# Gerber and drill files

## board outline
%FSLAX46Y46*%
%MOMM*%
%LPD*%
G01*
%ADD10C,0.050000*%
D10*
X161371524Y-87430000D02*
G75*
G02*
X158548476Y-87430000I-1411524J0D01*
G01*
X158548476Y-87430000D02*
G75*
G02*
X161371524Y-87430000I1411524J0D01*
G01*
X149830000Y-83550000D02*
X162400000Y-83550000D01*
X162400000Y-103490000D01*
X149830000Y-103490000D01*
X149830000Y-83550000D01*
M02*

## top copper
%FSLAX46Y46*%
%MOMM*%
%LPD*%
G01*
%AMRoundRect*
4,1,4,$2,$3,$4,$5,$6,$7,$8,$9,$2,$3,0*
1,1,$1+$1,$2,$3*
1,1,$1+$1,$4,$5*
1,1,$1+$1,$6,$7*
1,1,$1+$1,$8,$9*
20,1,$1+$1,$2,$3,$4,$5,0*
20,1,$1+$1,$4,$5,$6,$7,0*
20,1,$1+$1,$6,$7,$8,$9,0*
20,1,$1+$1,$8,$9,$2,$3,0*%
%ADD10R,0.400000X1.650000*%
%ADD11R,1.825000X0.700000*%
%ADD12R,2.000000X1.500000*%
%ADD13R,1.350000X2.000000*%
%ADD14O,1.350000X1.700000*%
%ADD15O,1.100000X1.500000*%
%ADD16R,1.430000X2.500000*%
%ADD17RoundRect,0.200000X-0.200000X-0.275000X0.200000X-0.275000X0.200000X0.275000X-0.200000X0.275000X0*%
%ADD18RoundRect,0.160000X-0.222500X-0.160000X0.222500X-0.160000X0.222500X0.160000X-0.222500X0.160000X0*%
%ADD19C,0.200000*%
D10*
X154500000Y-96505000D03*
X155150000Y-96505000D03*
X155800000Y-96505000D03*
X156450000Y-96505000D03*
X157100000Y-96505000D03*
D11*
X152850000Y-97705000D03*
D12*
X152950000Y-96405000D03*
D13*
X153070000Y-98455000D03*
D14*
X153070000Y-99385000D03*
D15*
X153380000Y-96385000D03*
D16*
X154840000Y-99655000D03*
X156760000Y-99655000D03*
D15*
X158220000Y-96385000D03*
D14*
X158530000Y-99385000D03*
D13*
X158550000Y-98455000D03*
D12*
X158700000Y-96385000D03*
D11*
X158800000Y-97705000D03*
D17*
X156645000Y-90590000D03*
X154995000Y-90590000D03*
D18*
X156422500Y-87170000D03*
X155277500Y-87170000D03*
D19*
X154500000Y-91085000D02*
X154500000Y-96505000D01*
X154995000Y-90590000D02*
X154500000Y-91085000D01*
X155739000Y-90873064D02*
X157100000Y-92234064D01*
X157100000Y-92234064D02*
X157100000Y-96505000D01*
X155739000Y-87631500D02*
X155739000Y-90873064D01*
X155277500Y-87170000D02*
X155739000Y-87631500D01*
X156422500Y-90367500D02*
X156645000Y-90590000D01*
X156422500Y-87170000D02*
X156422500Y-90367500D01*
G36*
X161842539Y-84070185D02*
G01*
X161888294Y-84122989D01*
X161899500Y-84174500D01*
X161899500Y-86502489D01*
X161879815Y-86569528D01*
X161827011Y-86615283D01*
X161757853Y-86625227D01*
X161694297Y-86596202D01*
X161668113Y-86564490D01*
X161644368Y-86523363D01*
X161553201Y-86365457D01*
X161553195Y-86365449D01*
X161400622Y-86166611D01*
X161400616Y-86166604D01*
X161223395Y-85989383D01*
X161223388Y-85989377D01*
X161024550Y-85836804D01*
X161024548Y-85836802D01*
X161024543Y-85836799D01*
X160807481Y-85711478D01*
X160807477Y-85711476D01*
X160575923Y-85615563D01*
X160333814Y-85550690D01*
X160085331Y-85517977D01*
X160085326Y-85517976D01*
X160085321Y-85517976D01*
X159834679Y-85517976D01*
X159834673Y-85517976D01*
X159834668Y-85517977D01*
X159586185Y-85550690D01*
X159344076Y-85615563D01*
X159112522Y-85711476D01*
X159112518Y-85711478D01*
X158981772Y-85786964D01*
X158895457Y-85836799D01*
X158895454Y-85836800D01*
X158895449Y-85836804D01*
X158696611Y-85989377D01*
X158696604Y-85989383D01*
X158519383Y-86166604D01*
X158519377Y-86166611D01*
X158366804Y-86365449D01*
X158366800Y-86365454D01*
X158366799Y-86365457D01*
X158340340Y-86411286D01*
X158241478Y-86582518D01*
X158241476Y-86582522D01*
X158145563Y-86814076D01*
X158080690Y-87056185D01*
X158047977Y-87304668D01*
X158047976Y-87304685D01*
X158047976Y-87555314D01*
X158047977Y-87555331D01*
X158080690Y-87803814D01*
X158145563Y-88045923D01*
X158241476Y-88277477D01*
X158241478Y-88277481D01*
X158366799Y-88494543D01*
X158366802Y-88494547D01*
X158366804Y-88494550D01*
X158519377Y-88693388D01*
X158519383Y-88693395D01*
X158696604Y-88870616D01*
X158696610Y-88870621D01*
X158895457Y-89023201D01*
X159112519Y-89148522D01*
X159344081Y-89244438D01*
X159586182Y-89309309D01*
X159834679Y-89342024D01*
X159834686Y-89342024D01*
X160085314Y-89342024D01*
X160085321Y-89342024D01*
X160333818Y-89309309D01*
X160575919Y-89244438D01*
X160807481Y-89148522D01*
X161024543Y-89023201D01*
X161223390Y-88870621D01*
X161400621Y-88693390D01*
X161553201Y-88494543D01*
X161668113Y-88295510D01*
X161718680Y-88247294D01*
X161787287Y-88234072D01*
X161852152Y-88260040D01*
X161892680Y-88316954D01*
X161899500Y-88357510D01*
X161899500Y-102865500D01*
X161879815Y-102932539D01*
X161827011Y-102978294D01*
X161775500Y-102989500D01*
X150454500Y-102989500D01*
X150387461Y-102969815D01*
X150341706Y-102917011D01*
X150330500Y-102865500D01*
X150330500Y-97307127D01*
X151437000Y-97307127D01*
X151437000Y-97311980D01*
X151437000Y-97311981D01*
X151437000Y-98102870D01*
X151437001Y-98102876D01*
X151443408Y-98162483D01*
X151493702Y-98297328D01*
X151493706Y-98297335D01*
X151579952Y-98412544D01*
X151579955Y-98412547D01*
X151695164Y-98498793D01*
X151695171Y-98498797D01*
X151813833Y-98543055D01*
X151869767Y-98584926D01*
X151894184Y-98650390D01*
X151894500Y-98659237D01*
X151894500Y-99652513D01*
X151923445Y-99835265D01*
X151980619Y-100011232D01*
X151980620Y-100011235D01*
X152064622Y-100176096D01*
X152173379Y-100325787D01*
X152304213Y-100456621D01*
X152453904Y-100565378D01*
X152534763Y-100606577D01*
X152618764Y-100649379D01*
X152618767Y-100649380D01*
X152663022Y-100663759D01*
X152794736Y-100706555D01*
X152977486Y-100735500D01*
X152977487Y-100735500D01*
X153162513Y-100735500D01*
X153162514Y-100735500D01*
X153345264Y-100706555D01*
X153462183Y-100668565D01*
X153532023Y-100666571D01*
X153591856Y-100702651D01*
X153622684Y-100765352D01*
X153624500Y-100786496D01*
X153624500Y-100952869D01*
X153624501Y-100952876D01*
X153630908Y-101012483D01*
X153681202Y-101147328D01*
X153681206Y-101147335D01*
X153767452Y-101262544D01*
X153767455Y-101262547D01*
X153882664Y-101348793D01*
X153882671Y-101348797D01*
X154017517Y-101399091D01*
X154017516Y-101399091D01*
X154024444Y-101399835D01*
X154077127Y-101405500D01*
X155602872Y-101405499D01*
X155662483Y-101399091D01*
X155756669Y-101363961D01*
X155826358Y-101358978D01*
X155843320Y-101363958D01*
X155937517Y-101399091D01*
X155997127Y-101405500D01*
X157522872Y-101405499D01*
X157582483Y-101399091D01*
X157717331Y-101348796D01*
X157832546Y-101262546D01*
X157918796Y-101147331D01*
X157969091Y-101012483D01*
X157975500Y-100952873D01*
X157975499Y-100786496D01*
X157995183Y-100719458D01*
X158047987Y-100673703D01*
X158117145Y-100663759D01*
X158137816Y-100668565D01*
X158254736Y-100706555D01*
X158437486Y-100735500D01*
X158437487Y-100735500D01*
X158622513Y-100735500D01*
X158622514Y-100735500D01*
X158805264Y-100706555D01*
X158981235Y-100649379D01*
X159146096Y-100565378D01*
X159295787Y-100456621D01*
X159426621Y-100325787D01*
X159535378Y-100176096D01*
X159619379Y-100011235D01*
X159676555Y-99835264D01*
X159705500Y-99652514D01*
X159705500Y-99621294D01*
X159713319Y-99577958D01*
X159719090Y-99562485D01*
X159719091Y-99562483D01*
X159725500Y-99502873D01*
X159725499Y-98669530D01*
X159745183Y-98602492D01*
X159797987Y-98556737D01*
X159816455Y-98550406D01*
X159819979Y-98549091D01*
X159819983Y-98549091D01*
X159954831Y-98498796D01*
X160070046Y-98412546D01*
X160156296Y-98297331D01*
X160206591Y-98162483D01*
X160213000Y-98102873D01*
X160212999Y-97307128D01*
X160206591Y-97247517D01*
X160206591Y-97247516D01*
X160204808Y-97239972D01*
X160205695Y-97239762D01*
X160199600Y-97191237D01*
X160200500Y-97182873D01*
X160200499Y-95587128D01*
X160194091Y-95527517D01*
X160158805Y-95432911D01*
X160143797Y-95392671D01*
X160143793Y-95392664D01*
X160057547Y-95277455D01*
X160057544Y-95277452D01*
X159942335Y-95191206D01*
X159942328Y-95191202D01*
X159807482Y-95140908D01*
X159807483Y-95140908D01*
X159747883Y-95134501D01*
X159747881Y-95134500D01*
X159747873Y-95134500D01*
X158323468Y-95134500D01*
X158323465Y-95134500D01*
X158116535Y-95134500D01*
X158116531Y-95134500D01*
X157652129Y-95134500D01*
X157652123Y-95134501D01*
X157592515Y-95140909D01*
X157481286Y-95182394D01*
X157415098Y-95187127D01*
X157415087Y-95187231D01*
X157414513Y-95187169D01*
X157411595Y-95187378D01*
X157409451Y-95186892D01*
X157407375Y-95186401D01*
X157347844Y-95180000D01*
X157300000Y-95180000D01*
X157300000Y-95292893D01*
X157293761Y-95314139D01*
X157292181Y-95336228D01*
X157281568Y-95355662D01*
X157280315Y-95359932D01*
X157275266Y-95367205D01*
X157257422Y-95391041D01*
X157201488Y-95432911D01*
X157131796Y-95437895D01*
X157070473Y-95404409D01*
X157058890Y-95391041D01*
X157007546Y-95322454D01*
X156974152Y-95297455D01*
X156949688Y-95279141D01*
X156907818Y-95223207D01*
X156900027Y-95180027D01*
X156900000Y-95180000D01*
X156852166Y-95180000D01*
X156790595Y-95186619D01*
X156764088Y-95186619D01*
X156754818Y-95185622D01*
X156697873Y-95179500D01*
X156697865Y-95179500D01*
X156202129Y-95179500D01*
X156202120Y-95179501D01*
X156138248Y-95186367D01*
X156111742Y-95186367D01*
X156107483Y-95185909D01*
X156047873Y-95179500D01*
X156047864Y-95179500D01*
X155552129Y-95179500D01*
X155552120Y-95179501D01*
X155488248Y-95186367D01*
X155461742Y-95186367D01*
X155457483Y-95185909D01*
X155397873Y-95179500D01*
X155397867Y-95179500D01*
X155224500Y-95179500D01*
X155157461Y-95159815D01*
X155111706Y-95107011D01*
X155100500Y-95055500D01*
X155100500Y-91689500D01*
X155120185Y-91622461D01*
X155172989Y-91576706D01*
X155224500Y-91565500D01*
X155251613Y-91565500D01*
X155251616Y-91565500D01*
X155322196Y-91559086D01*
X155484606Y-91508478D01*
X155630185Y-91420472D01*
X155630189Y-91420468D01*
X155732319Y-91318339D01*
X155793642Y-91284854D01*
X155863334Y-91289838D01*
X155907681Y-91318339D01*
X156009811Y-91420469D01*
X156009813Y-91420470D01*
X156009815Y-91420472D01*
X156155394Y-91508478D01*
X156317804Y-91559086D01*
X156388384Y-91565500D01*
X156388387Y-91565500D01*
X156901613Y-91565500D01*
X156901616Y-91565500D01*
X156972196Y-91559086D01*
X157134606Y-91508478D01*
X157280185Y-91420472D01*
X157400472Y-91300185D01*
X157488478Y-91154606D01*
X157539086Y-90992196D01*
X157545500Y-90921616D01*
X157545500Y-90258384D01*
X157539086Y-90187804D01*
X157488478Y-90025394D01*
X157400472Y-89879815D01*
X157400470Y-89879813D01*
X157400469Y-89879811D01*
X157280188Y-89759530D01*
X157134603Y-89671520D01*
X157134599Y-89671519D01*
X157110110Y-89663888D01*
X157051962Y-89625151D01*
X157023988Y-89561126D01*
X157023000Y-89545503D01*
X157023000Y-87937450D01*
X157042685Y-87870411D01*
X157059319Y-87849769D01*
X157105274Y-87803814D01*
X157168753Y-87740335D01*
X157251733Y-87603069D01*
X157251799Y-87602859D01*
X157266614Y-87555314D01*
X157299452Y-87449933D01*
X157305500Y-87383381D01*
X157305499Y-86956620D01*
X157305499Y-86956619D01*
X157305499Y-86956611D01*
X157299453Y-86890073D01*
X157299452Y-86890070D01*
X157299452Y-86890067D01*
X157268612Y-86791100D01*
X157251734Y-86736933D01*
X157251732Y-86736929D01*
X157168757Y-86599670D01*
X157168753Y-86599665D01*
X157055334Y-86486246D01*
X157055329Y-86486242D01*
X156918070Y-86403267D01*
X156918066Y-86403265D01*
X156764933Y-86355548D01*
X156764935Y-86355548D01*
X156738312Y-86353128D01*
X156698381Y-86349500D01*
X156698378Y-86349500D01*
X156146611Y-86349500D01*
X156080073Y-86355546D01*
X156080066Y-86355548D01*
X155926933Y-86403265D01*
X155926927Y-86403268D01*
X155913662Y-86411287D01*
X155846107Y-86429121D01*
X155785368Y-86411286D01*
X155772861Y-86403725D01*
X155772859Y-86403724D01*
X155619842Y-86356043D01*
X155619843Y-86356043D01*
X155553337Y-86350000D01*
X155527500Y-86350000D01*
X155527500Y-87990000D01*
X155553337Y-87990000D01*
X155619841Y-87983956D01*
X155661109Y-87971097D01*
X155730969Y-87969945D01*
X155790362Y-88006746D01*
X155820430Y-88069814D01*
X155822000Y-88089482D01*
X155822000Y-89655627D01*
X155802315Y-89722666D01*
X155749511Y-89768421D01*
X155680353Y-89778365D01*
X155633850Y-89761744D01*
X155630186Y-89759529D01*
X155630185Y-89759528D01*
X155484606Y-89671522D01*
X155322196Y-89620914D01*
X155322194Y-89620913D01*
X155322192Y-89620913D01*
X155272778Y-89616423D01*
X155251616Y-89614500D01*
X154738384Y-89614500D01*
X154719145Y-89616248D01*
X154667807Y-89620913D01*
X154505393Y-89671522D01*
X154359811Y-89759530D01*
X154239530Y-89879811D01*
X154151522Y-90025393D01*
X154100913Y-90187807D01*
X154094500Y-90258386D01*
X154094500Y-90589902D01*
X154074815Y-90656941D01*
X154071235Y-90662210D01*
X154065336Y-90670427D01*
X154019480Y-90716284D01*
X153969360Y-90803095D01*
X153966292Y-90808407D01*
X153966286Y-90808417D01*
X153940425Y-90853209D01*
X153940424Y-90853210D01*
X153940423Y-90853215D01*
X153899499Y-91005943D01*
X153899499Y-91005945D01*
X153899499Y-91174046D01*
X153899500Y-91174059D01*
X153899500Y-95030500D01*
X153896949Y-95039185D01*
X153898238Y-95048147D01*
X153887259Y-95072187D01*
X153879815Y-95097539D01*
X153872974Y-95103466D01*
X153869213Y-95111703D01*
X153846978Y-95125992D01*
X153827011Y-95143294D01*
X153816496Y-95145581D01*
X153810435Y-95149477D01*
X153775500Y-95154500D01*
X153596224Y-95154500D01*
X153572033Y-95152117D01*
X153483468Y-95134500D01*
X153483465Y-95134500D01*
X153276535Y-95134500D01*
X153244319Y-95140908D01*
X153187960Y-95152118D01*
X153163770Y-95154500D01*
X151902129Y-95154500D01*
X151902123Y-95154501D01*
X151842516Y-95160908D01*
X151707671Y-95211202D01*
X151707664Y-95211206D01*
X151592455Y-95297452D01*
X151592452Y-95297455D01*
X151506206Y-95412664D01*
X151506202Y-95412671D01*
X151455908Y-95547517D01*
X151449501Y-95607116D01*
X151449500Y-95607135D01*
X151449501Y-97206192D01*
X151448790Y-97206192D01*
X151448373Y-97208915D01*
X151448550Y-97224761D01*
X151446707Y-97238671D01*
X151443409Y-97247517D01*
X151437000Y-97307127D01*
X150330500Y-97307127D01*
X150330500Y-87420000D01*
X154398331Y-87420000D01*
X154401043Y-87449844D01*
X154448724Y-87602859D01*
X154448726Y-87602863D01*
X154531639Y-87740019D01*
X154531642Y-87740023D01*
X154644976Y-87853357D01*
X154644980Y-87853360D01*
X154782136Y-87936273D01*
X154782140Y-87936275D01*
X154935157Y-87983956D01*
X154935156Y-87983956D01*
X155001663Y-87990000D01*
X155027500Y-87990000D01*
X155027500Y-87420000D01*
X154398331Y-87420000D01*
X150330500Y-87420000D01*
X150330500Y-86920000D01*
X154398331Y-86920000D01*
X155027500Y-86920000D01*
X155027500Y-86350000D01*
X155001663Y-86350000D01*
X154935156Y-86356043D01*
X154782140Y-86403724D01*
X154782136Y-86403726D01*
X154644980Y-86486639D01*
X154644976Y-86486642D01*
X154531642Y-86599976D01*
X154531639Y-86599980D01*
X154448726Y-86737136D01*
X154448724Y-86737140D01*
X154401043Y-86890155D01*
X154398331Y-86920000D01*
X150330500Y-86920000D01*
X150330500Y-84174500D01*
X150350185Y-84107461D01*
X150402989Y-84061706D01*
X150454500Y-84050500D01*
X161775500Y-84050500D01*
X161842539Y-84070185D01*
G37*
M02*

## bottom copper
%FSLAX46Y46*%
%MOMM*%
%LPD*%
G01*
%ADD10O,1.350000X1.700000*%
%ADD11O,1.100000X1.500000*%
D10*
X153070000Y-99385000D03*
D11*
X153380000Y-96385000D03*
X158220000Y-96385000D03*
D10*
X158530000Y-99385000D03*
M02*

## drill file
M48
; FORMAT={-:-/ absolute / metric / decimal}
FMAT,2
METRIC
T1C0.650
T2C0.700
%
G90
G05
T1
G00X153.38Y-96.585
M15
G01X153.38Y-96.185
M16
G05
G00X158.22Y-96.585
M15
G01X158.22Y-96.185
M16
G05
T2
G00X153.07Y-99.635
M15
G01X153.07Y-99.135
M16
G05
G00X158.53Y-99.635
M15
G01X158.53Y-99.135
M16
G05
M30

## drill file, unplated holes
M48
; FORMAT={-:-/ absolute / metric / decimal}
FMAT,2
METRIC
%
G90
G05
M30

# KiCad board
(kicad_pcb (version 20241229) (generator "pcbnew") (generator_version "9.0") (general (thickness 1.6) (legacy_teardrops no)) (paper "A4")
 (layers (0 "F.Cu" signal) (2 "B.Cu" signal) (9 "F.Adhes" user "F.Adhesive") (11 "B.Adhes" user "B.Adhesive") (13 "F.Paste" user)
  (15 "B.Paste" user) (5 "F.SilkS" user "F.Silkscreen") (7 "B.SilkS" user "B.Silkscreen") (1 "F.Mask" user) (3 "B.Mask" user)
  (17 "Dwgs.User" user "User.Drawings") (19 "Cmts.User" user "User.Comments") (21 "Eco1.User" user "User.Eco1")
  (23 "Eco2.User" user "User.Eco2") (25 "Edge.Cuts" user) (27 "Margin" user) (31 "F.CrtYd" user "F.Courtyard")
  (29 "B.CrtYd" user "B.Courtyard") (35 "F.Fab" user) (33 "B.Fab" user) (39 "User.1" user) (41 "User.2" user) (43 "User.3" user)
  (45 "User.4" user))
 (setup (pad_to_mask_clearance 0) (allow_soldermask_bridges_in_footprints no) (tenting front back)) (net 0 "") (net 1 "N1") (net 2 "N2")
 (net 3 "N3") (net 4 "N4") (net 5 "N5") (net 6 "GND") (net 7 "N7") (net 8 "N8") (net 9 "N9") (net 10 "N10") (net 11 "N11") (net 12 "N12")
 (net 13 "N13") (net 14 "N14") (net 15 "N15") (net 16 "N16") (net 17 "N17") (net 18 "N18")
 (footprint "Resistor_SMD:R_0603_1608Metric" (layer "F.Cu") (at 155.82 90.59)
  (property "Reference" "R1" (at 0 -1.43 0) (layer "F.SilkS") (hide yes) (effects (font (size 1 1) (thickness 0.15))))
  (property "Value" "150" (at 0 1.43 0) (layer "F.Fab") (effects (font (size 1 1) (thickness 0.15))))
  (pad "1" smd roundrect (at -0.825 0) (size 0.8 0.95) (layers "F.Cu" "F.Mask" "F.Paste") (roundrect_rratio 0.25) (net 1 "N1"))
  (pad "2" smd roundrect (at 0.825 0) (size 0.8 0.95) (layers "F.Cu" "F.Mask" "F.Paste") (roundrect_rratio 0.25) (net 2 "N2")))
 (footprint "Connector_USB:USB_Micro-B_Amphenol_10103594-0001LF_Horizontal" (layer "F.Cu") (at 155.825 98.27)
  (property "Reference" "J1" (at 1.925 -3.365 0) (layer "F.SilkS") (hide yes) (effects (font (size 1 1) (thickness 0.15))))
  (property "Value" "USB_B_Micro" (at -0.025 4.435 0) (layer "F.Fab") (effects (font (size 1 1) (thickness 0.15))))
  (pad "1" smd rect (at -1.325 -1.765 90) (size 1.65 0.4) (layers "F.Cu" "F.Mask" "F.Paste") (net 1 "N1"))
  (pad "2" smd rect (at -0.675 -1.765 90) (size 1.65 0.4) (layers "F.Cu" "F.Mask" "F.Paste") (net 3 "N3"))
  (pad "3" smd rect (at -0.025 -1.765 90) (size 1.65 0.4) (layers "F.Cu" "F.Mask" "F.Paste") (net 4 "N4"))
  (pad "4" smd rect (at 0.625 -1.765 90) (size 1.65 0.4) (layers "F.Cu" "F.Mask" "F.Paste") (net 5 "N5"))
  (pad "5" smd rect (at 1.275 -1.765 90) (size 1.65 0.4) (layers "F.Cu" "F.Mask" "F.Paste") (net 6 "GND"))
  (pad "6" smd rect (at -2.975 -0.565) (size 1.825 0.7) (layers "F.Cu" "F.Mask" "F.Paste") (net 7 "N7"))
  (pad "6" smd rect (at -2.875 -1.865) (size 2 1.5) (layers "F.Cu" "F.Mask" "F.Paste") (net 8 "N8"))
  (pad "6" smd rect (at -2.755 0.185) (size 1.35 2) (layers "F.Cu" "F.Mask" "F.Paste") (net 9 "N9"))
  (pad "6" thru_hole oval (at -2.755 1.115 90) (size 1.7 1.35) (drill oval 1.2 0.7) (layers "*.Cu" "*.Mask") (remove_unused_layers no)
   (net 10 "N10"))
  (pad "6" thru_hole oval (at -2.445 -1.885 90) (size 1.5 1.1) (drill oval 1.05 0.65) (layers "*.Cu" "*.Mask") (remove_unused_layers no)
   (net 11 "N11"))
  (pad "6" smd rect (at -0.985 1.385 90) (size 2.5 1.43) (layers "F.Cu" "F.Mask" "F.Paste") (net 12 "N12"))
  (pad "6" smd rect (at 0.935 1.385 90) (size 2.5 1.43) (layers "F.Cu" "F.Mask" "F.Paste") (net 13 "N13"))
  (pad "6" thru_hole oval (at 2.395 -1.885 90) (size 1.5 1.1) (drill oval 1.05 0.65) (layers "*.Cu" "*.Mask") (remove_unused_layers no)
   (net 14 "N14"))
  (pad "6" thru_hole oval (at 2.705 1.115 90) (size 1.7 1.35) (drill oval 1.2 0.7) (layers "*.Cu" "*.Mask") (remove_unused_layers no)
   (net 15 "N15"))
  (pad "6" smd rect (at 2.725 0.185) (size 1.35 2) (layers "F.Cu" "F.Mask" "F.Paste") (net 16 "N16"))
  (pad "6" smd rect (at 2.875 -1.885) (size 2 1.5) (layers "F.Cu" "F.Mask" "F.Paste") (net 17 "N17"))
  (pad "6" smd rect (at 2.975 -0.565) (size 1.825 0.7) (layers "F.Cu" "F.Mask" "F.Paste") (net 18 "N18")))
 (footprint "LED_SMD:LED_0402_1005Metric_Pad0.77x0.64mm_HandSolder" (layer "F.Cu") (at 155.85 87.17)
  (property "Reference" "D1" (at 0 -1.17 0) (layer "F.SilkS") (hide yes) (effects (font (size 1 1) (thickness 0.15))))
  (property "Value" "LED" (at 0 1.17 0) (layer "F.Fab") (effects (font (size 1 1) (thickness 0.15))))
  (pad "1" smd roundrect (at -0.5725 0) (size 0.765 0.64) (layers "F.Cu" "F.Mask" "F.Paste") (roundrect_rratio 0.25) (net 6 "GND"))
  (pad "2" smd roundrect (at 0.5725 0) (size 0.765 0.64) (layers "F.Cu" "F.Mask" "F.Paste") (roundrect_rratio 0.25) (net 2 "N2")))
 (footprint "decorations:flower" (layer "F.Cu") (at 153.961703 91.14243)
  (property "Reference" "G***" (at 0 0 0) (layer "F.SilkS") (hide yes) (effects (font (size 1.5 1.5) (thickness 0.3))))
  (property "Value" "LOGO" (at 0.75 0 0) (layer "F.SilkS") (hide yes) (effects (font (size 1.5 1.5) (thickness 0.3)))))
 (gr_circle (center 159.96 87.43) (end 160.14 88.83) (stroke (width 0.05) (type default)) (fill no) (layer "Edge.Cuts"))
 (gr_rect (start 149.83 83.55) (end 162.4 103.49) (stroke (width 0.05) (type default)) (fill no) (layer "Edge.Cuts"))
 (segment (start 156.4225 90.3675) (end 156.645 90.59) (width 0.2) (layer "F.Cu") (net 2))
 (segment (start 156.4225 87.17) (end 156.4225 90.3675) (width 0.2) (layer "F.Cu") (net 2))
 (segment (start 157.1 92.234064) (end 157.1 96.505) (width 0.2) (layer "F.Cu") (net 6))
 (segment (start 155.739 90.873064) (end 157.1 92.234064) (width 0.2) (layer "F.Cu") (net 6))
 (segment (start 155.739 87.6315) (end 155.739 90.873064) (width 0.2) (layer "F.Cu") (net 6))
 (segment (start 155.2775 87.17) (end 155.739 87.6315) (width 0.2) (layer "F.Cu") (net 6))
 (segment (start 154.995 90.59) (end 154.5 91.085) (width 0.2) (layer "F.Cu") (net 1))
 (segment (start 154.5 91.085) (end 154.5 96.505) (width 0.2) (layer "F.Cu") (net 1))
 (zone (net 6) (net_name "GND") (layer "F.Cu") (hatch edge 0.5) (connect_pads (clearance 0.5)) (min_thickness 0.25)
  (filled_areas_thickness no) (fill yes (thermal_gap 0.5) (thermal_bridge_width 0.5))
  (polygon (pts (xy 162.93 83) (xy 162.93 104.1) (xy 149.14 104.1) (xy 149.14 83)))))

